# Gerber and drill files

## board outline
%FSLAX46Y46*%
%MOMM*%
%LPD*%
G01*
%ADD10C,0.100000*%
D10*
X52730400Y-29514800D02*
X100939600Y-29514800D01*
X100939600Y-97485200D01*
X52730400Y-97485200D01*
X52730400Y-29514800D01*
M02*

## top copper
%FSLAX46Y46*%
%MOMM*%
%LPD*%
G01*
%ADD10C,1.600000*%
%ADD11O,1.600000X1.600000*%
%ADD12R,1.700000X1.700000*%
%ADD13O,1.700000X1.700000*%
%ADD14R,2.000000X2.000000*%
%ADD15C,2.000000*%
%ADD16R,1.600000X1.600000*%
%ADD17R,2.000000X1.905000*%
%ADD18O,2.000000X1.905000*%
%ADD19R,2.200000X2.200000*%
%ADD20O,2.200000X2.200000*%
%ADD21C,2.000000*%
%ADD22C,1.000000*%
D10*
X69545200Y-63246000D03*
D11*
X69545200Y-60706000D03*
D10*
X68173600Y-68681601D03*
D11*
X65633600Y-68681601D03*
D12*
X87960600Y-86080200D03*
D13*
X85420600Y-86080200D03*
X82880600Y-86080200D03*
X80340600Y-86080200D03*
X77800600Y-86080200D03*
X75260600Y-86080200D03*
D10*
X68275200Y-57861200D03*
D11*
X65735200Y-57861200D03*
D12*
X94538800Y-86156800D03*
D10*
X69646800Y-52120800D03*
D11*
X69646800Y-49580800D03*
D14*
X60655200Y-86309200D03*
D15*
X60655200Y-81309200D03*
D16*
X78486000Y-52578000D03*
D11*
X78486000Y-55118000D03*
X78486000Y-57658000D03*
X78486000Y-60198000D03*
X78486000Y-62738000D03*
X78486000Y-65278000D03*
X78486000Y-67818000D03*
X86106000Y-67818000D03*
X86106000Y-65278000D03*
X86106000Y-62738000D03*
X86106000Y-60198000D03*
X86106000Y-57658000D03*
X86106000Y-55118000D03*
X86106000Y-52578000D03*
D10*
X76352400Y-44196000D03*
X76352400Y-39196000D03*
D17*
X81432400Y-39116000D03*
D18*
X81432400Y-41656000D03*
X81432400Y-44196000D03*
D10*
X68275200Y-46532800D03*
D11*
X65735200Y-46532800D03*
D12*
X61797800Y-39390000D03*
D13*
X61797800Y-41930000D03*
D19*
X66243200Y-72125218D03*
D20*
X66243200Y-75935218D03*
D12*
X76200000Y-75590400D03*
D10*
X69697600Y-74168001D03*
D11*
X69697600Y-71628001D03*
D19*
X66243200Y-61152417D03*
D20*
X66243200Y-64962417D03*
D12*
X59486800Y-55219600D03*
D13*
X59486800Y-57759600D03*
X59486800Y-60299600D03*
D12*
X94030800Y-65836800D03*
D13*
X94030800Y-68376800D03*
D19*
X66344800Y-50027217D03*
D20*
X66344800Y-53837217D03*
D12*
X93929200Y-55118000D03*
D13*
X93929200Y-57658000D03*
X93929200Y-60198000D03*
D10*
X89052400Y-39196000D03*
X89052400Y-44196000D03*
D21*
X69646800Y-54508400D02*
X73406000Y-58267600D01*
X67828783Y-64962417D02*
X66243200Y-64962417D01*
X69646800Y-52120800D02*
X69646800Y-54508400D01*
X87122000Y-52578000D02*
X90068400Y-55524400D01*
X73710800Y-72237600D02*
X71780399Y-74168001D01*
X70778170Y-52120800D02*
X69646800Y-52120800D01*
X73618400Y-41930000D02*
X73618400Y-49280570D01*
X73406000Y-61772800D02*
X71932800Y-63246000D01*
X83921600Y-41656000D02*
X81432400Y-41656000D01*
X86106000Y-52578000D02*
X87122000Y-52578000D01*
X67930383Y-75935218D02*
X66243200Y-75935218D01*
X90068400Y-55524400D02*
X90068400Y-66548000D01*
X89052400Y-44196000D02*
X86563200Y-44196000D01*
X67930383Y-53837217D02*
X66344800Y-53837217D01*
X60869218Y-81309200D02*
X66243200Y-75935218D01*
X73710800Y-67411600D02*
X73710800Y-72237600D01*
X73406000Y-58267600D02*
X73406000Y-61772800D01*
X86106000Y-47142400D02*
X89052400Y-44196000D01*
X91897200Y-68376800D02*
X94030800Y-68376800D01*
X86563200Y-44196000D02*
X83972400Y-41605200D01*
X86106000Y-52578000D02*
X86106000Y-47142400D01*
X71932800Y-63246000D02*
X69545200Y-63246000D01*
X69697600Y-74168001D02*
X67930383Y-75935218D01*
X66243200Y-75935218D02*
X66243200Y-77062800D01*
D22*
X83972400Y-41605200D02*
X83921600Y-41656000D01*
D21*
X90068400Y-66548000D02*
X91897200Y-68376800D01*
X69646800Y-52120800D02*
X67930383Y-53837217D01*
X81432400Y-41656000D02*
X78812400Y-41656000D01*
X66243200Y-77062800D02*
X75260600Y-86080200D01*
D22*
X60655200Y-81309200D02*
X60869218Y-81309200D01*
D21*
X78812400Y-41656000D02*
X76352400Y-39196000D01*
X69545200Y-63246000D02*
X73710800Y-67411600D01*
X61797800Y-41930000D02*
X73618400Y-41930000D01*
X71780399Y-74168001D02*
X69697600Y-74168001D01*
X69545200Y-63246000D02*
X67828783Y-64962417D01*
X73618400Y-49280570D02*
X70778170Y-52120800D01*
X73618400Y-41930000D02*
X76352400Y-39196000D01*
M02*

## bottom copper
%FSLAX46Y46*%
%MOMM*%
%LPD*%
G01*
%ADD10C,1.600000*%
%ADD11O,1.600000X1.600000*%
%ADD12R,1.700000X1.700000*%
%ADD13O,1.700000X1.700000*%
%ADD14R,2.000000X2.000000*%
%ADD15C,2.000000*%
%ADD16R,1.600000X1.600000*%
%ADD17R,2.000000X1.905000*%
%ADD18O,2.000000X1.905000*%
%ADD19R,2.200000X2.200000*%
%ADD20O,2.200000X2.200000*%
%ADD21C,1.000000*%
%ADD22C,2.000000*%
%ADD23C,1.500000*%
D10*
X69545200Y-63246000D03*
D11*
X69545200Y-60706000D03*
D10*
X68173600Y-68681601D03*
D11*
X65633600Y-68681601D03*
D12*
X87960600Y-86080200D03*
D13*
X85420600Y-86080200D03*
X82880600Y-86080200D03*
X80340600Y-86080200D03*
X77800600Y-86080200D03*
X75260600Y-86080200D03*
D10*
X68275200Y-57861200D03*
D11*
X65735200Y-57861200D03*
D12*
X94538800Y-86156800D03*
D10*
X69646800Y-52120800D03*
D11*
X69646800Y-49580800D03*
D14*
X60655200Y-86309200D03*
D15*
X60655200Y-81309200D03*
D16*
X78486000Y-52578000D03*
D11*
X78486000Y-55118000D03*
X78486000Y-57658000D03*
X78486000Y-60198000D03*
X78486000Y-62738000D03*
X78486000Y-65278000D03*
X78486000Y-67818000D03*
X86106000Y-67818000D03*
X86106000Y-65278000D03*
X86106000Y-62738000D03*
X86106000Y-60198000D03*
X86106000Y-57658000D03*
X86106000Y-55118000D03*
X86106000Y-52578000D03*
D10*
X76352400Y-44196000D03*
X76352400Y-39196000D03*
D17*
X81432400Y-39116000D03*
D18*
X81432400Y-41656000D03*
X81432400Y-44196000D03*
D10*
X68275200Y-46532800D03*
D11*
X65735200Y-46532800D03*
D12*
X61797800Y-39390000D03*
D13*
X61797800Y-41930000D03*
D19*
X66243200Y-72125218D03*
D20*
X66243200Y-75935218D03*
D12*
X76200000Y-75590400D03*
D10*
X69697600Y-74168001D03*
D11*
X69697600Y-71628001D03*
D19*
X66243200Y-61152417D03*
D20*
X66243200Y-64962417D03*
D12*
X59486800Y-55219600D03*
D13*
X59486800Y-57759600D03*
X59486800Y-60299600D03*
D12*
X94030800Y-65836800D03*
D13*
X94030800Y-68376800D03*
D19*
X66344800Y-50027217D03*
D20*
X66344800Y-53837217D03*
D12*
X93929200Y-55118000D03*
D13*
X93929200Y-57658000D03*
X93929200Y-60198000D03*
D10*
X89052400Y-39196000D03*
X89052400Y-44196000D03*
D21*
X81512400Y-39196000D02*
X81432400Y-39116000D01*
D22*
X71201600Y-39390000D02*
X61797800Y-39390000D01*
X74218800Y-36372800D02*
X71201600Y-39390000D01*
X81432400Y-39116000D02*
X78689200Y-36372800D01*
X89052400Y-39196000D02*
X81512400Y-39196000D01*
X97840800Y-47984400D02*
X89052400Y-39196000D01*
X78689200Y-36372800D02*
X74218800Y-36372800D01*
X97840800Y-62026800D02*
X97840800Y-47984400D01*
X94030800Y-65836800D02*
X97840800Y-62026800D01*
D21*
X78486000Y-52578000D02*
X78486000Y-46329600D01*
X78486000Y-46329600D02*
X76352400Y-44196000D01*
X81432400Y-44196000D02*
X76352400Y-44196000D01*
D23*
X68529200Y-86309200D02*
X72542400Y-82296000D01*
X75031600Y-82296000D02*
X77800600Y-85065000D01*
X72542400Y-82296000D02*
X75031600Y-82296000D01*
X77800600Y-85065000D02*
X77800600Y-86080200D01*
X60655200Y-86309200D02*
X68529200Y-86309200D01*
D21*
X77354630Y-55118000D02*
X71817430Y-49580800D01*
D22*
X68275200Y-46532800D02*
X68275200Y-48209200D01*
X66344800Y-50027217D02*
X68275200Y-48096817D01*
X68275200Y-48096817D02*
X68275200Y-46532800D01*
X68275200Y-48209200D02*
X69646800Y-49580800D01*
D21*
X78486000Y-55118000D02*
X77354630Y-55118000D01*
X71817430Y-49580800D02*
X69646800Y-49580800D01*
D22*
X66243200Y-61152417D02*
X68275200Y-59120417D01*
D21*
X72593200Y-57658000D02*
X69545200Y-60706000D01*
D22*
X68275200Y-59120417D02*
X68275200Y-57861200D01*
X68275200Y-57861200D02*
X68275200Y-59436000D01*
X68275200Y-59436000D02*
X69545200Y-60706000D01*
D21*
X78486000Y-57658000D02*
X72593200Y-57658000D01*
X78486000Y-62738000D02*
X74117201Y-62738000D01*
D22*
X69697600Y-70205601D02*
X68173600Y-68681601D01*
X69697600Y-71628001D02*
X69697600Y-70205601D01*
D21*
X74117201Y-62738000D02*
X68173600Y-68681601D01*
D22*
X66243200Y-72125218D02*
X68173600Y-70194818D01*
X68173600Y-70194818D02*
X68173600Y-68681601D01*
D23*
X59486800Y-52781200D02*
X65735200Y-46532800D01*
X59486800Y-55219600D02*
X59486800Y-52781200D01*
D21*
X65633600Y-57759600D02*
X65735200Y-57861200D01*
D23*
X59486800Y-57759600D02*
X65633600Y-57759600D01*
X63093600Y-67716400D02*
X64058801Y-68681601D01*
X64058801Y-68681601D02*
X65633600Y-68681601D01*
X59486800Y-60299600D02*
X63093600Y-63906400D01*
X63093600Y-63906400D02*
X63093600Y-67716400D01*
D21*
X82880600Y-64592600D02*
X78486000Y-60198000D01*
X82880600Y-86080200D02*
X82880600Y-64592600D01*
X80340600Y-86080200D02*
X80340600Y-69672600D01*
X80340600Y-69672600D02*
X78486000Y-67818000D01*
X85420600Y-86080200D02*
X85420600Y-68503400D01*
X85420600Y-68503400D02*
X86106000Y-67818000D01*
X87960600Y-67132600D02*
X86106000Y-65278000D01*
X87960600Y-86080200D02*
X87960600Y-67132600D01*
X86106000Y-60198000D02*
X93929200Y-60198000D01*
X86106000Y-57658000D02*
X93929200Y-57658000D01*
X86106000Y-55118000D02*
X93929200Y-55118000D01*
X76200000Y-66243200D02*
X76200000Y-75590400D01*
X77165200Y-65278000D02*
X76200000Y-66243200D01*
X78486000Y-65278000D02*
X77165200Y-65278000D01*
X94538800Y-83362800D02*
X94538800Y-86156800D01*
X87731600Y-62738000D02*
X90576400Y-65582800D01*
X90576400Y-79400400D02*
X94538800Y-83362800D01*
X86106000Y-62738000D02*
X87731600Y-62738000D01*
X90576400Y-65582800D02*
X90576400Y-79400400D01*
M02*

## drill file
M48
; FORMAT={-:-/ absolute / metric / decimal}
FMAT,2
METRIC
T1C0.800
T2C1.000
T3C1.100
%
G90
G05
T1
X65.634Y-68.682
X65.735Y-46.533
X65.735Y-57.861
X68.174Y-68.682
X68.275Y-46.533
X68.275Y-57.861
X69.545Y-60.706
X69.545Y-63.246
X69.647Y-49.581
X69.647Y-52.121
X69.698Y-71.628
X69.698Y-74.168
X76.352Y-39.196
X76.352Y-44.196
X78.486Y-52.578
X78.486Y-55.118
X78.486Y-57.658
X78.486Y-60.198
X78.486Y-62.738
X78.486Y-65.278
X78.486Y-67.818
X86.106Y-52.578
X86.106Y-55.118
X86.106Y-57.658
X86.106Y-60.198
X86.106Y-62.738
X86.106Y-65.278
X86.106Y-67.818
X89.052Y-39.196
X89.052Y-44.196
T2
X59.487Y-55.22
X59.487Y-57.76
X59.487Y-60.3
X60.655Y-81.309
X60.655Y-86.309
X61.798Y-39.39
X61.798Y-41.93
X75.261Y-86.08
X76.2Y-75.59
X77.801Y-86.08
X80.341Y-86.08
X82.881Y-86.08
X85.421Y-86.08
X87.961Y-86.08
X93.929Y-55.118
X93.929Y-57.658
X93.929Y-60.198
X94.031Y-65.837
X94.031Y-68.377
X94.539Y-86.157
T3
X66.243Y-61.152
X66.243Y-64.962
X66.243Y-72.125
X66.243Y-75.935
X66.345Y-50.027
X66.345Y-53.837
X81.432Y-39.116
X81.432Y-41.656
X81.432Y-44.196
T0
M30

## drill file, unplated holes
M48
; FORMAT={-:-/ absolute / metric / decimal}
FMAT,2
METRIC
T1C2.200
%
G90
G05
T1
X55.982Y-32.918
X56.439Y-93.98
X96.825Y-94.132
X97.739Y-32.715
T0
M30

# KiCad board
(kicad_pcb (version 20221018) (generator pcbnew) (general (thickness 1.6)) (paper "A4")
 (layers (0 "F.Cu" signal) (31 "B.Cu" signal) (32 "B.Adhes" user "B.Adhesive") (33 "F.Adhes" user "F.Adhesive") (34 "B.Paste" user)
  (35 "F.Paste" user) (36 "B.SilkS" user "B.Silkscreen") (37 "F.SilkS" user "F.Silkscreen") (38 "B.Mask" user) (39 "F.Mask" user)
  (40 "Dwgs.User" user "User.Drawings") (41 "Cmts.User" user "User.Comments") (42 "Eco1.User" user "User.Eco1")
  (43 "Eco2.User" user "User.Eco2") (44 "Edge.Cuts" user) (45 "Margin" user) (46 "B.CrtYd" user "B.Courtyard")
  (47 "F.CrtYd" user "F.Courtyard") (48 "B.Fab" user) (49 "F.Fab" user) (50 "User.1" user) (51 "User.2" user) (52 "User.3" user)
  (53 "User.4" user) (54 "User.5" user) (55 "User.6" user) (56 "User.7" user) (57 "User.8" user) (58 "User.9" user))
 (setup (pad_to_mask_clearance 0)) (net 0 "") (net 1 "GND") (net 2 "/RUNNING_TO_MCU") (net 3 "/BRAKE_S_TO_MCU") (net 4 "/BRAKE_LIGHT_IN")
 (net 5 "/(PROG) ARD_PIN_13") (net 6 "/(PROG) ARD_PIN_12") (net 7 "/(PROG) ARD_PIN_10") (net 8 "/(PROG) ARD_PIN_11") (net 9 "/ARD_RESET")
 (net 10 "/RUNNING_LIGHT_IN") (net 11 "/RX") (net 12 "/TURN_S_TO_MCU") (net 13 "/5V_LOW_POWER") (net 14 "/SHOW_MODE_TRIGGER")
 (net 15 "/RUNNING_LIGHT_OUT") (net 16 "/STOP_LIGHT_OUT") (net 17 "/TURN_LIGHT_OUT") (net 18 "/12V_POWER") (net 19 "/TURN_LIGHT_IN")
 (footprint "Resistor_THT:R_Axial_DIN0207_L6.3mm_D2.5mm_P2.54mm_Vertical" (layer "F.Cu") (at 69.5452 63.246 90)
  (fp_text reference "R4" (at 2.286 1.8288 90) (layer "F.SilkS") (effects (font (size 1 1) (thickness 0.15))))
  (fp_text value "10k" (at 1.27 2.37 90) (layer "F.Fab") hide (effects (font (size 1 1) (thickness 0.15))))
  (pad "1" thru_hole circle (at 0 0 90) (size 1.6 1.6) (drill 0.8) (layers "*.Cu" "*.Mask") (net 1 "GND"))
  (pad "2" thru_hole oval (at 2.54 0 90) (size 1.6 1.6) (drill 0.8) (layers "*.Cu" "*.Mask") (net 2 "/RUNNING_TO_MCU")))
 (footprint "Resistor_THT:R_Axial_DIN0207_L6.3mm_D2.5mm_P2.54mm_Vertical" (layer "F.Cu") (at 68.1736 68.681601 180)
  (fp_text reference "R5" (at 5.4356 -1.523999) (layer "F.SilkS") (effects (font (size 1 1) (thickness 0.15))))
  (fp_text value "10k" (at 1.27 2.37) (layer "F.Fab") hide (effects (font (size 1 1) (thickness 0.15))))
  (pad "1" thru_hole circle (at 0 0 180) (size 1.6 1.6) (drill 0.8) (layers "*.Cu" "*.Mask") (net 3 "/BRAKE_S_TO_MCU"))
  (pad "2" thru_hole oval (at 2.54 0 180) (size 1.6 1.6) (drill 0.8) (layers "*.Cu" "*.Mask") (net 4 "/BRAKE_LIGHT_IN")))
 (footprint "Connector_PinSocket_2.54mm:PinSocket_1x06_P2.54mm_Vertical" (layer "F.Cu") (at 87.9606 86.0802 -90)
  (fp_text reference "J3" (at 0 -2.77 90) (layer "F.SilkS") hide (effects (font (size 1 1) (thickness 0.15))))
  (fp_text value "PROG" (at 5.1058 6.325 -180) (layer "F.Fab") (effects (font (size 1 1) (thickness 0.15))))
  (pad "1" thru_hole rect (at 0 0 270) (size 1.7 1.7) (drill 1) (layers "*.Cu" "*.Mask") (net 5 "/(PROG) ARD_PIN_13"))
  (pad "2" thru_hole oval (at 0 2.54 270) (size 1.7 1.7) (drill 1) (layers "*.Cu" "*.Mask") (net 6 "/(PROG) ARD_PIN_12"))
  (pad "3" thru_hole oval (at 0 5.08 270) (size 1.7 1.7) (drill 1) (layers "*.Cu" "*.Mask") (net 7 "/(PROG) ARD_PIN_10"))
  (pad "4" thru_hole oval (at 0 7.62 270) (size 1.7 1.7) (drill 1) (layers "*.Cu" "*.Mask") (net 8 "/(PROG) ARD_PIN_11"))
  (pad "5" thru_hole oval (at 0 10.16 270) (size 1.7 1.7) (drill 1) (layers "*.Cu" "*.Mask") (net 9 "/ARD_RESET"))
  (pad "6" thru_hole oval (at 0 12.7 270) (size 1.7 1.7) (drill 1) (layers "*.Cu" "*.Mask") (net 1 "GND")))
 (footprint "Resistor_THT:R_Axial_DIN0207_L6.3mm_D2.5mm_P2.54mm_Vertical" (layer "F.Cu") (at 68.2752 57.8612 180)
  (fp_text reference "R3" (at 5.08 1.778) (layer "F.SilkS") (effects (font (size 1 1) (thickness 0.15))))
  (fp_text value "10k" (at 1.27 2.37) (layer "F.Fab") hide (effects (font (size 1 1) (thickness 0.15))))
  (pad "1" thru_hole circle (at 0 0 180) (size 1.6 1.6) (drill 0.8) (layers "*.Cu" "*.Mask") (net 2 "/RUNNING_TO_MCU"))
  (pad "2" thru_hole oval (at 2.54 0 180) (size 1.6 1.6) (drill 0.8) (layers "*.Cu" "*.Mask") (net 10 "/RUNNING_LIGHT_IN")))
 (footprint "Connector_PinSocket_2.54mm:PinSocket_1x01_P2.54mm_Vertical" (layer "F.Cu") (at 94.5388 86.1568)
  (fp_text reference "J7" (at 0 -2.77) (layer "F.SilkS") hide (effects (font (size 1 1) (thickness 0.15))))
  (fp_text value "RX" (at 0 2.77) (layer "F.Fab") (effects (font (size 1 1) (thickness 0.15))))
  (pad "1" thru_hole rect (at 0 0) (size 1.7 1.7) (drill 1) (layers "*.Cu" "*.Mask") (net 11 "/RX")))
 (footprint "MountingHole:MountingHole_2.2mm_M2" (layer "F.Cu") (at 96.8248 94.1324)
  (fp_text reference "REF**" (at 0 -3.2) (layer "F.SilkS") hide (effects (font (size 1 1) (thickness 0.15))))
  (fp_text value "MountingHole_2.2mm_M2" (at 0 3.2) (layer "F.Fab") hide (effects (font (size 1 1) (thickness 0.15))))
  (pad "" np_thru_hole circle (at 0 0) (size 2.2 2.2) (drill 2.2) (layers "*.Cu" "*.Mask")))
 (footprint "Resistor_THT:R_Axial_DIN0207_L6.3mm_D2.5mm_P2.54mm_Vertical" (layer "F.Cu") (at 69.6468 52.1208 90)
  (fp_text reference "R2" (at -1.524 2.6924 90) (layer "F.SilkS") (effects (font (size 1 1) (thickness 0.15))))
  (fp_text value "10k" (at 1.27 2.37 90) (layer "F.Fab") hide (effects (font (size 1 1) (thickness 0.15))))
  (pad "1" thru_hole circle (at 0 0 90) (size 1.6 1.6) (drill 0.8) (layers "*.Cu" "*.Mask") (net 1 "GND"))
  (pad "2" thru_hole oval (at 2.54 0 90) (size 1.6 1.6) (drill 0.8) (layers "*.Cu" "*.Mask") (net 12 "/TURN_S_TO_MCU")))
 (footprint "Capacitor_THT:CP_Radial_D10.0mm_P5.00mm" (layer "F.Cu") (at 60.6552 86.3092 90)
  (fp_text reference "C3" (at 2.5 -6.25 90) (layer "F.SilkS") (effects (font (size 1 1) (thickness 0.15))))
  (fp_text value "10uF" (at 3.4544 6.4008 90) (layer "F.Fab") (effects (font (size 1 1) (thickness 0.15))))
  (pad "1" thru_hole rect (at 0 0 90) (size 2 2) (drill 1) (layers "*.Cu" "*.Mask") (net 9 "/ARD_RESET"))
  (pad "2" thru_hole circle (at 5 0 90) (size 2 2) (drill 1) (layers "*.Cu" "*.Mask") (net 1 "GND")))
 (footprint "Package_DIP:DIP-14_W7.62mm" (layer "F.Cu") (at 78.486 52.578)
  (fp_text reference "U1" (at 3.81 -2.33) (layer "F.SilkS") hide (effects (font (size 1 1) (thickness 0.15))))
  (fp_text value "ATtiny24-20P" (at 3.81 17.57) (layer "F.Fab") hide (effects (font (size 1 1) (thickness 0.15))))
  (pad "1" thru_hole rect (at 0 0) (size 1.6 1.6) (drill 0.8) (layers "*.Cu" "*.Mask") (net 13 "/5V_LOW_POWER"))
  (pad "2" thru_hole oval (at 0 2.54) (size 1.6 1.6) (drill 0.8) (layers "*.Cu" "*.Mask") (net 12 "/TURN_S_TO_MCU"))
  (pad "3" thru_hole oval (at 0 5.08) (size 1.6 1.6) (drill 0.8) (layers "*.Cu" "*.Mask") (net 2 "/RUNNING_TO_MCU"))
  (pad "4" thru_hole oval (at 0 7.62) (size 1.6 1.6) (drill 0.8) (layers "*.Cu" "*.Mask") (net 7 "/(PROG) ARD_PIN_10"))
  (pad "5" thru_hole oval (at 0 10.16) (size 1.6 1.6) (drill 0.8) (layers "*.Cu" "*.Mask") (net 3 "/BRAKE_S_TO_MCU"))
  (pad "6" thru_hole oval (at 0 12.7) (size 1.6 1.6) (drill 0.8) (layers "*.Cu" "*.Mask") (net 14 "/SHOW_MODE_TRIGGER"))
  (pad "7" thru_hole oval (at 0 15.24) (size 1.6 1.6) (drill 0.8) (layers "*.Cu" "*.Mask") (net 8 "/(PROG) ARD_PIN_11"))
  (pad "8" thru_hole oval (at 7.62 15.24) (size 1.6 1.6) (drill 0.8) (layers "*.Cu" "*.Mask") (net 6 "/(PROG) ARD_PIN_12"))
  (pad "9" thru_hole oval (at 7.62 12.7) (size 1.6 1.6) (drill 0.8) (layers "*.Cu" "*.Mask") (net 5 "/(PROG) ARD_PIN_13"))
  (pad "10" thru_hole oval (at 7.62 10.16) (size 1.6 1.6) (drill 0.8) (layers "*.Cu" "*.Mask") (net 11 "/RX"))
  (pad "11" thru_hole oval (at 7.62 7.62) (size 1.6 1.6) (drill 0.8) (layers "*.Cu" "*.Mask") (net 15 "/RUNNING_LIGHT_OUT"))
  (pad "12" thru_hole oval (at 7.62 5.08) (size 1.6 1.6) (drill 0.8) (layers "*.Cu" "*.Mask") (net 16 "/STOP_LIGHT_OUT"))
  (pad "13" thru_hole oval (at 7.62 2.54) (size 1.6 1.6) (drill 0.8) (layers "*.Cu" "*.Mask") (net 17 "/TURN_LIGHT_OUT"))
  (pad "14" thru_hole oval (at 7.62 0) (size 1.6 1.6) (drill 0.8) (layers "*.Cu" "*.Mask") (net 1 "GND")))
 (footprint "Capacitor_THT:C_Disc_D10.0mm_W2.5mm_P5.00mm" (layer "F.Cu") (at 76.3524 44.196 90)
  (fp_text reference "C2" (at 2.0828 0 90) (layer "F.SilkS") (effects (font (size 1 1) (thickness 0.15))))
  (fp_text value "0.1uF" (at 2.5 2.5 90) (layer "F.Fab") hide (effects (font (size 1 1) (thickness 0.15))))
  (pad "1" thru_hole circle (at 0 0 90) (size 1.6 1.6) (drill 0.8) (layers "*.Cu" "*.Mask") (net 13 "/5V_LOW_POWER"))
  (pad "2" thru_hole circle (at 5 0 90) (size 1.6 1.6) (drill 0.8) (layers "*.Cu" "*.Mask") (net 1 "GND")))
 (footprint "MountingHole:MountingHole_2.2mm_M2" (layer "F.Cu") (at 56.4388 93.98)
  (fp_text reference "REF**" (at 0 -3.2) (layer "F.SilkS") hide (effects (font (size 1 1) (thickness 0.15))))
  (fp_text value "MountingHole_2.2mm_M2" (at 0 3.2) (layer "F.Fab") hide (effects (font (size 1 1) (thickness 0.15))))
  (pad "" np_thru_hole circle (at 0 0) (size 2.2 2.2) (drill 2.2) (layers "*.Cu" "*.Mask")))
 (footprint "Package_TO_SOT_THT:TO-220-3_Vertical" (layer "F.Cu") (at 81.4324 39.116 -90)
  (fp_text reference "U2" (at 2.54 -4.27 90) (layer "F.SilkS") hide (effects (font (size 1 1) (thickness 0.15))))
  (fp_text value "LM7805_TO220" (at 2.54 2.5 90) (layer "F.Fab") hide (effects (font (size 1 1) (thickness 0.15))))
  (pad "1" thru_hole rect (at 0 0 270) (size 1.905 2) (drill 1.1) (layers "*.Cu" "*.Mask") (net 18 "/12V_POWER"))
  (pad "2" thru_hole oval (at 2.54 0 270) (size 1.905 2) (drill 1.1) (layers "*.Cu" "*.Mask") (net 1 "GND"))
  (pad "3" thru_hole oval (at 5.08 0 270) (size 1.905 2) (drill 1.1) (layers "*.Cu" "*.Mask") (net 13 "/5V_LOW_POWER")))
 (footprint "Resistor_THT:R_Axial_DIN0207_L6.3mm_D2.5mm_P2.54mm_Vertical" (layer "F.Cu") (at 68.2752 46.5328 180)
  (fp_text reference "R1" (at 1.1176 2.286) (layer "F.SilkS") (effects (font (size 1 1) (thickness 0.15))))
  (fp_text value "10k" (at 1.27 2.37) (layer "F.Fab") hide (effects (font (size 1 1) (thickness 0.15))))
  (pad "1" thru_hole circle (at 0 0 180) (size 1.6 1.6) (drill 0.8) (layers "*.Cu" "*.Mask") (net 12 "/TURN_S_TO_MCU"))
  (pad "2" thru_hole oval (at 2.54 0 180) (size 1.6 1.6) (drill 0.8) (layers "*.Cu" "*.Mask") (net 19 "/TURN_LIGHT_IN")))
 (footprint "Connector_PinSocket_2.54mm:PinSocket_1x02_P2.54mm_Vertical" (layer "F.Cu") (at 61.7978 39.39)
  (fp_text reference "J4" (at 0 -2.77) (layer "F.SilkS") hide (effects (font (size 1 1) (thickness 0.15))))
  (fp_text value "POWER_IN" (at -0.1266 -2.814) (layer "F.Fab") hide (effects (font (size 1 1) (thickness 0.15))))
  (pad "1" thru_hole rect (at 0 0) (size 1.7 1.7) (drill 1) (layers "*.Cu" "*.Mask") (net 18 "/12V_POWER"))
  (pad "2" thru_hole oval (at 0 2.54) (size 1.7 1.7) (drill 1) (layers "*.Cu" "*.Mask") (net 1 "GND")))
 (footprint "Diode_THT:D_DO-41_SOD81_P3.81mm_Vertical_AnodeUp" (layer "F.Cu") (at 66.2432 72.125218 -90)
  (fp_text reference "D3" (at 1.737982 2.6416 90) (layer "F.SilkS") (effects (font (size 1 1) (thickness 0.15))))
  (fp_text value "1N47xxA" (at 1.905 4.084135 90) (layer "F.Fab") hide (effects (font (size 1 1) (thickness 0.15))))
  (pad "1" thru_hole rect (at 0 0 270) (size 2.2 2.2) (drill 1.1) (layers "*.Cu" "*.Mask") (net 3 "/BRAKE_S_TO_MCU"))
  (pad "2" thru_hole oval (at 3.81 0 270) (size 2.2 2.2) (drill 1.1) (layers "*.Cu" "*.Mask") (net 1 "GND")))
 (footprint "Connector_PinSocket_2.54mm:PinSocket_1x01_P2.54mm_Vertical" (layer "F.Cu") (at 76.2 75.5904)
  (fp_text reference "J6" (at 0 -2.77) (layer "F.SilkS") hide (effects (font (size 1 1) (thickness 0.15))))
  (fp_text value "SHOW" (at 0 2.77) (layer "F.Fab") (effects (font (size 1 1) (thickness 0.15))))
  (pad "1" thru_hole rect (at 0 0) (size 1.7 1.7) (drill 1) (layers "*.Cu" "*.Mask") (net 14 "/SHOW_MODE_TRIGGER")))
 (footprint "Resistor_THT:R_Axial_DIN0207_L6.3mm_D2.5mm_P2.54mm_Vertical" (layer "F.Cu") (at 69.6976 74.168001 90)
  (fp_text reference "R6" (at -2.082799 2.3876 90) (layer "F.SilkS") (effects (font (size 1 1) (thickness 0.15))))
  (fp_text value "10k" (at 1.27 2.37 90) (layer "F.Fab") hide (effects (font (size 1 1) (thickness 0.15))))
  (pad "1" thru_hole circle (at 0 0 90) (size 1.6 1.6) (drill 0.8) (layers "*.Cu" "*.Mask") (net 1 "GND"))
  (pad "2" thru_hole oval (at 2.54 0 90) (size 1.6 1.6) (drill 0.8) (layers "*.Cu" "*.Mask") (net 3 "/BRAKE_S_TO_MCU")))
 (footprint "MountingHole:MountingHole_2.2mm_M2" (layer "F.Cu") (at 55.9816 32.9184)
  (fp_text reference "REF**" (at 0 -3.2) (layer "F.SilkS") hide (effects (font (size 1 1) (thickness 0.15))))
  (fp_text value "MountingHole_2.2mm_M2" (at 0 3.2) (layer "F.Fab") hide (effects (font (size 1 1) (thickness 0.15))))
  (pad "" np_thru_hole circle (at 0 0) (size 2.2 2.2) (drill 2.2) (layers "*.Cu" "*.Mask")))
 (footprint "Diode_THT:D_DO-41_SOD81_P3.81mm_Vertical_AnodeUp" (layer "F.Cu") (at 66.2432 61.152417 -90)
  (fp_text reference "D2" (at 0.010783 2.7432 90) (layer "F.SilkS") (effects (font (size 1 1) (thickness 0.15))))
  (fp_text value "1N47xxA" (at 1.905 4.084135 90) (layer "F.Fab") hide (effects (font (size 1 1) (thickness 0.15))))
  (pad "1" thru_hole rect (at 0 0 270) (size 2.2 2.2) (drill 1.1) (layers "*.Cu" "*.Mask") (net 2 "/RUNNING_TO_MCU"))
  (pad "2" thru_hole oval (at 3.81 0 270) (size 2.2 2.2) (drill 1.1) (layers "*.Cu" "*.Mask") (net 1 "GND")))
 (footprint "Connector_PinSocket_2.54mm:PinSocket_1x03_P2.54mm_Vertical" (layer "F.Cu") (at 59.4868 55.2196)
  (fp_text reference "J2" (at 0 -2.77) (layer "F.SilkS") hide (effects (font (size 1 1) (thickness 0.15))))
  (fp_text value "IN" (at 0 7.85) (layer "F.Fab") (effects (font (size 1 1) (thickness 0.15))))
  (pad "1" thru_hole rect (at 0 0) (size 1.7 1.7) (drill 1) (layers "*.Cu" "*.Mask") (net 19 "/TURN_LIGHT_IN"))
  (pad "2" thru_hole oval (at 0 2.54) (size 1.7 1.7) (drill 1) (layers "*.Cu" "*.Mask") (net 10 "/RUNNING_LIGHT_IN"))
  (pad "3" thru_hole oval (at 0 5.08) (size 1.7 1.7) (drill 1) (layers "*.Cu" "*.Mask") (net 4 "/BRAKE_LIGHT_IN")))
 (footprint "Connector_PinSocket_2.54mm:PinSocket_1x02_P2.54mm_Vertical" (layer "F.Cu") (at 94.0308 65.8368)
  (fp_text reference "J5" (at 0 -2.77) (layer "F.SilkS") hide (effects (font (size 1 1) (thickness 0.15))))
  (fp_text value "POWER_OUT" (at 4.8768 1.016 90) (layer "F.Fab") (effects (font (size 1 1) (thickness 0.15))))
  (pad "1" thru_hole rect (at 0 0) (size 1.7 1.7) (drill 1) (layers "*.Cu" "*.Mask") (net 18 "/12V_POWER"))
  (pad "2" thru_hole oval (at 0 2.54) (size 1.7 1.7) (drill 1) (layers "*.Cu" "*.Mask") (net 1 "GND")))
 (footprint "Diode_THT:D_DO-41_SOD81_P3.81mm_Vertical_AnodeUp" (layer "F.Cu") (at 66.3448 50.027217 -90)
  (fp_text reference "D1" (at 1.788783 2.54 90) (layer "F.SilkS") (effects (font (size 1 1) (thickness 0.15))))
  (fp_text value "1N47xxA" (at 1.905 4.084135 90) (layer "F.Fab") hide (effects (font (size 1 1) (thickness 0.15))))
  (pad "1" thru_hole rect (at 0 0 270) (size 2.2 2.2) (drill 1.1) (layers "*.Cu" "*.Mask") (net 12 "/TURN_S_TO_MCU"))
  (pad "2" thru_hole oval (at 3.81 0 270) (size 2.2 2.2) (drill 1.1) (layers "*.Cu" "*.Mask") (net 1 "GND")))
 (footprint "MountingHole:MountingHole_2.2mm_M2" (layer "F.Cu") (at 97.7392 32.7152)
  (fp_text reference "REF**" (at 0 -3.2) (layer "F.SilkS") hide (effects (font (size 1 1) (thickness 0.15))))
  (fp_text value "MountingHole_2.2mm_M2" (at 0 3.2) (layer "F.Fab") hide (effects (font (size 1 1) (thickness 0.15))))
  (pad "" np_thru_hole circle (at 0 0) (size 2.2 2.2) (drill 2.2) (layers "*.Cu" "*.Mask")))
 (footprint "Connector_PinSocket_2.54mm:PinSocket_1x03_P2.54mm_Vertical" (layer "F.Cu") (at 93.9292 55.118)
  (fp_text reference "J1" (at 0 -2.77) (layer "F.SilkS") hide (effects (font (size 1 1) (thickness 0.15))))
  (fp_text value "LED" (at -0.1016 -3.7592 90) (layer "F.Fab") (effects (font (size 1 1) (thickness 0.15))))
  (pad "1" thru_hole rect (at 0 0) (size 1.7 1.7) (drill 1) (layers "*.Cu" "*.Mask") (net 17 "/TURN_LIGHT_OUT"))
  (pad "2" thru_hole oval (at 0 2.54) (size 1.7 1.7) (drill 1) (layers "*.Cu" "*.Mask") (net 16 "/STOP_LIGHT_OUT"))
  (pad "3" thru_hole oval (at 0 5.08) (size 1.7 1.7) (drill 1) (layers "*.Cu" "*.Mask") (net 15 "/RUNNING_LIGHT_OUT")))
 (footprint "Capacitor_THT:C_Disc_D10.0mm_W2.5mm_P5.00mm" (layer "F.Cu") (at 89.0524 39.196 -90)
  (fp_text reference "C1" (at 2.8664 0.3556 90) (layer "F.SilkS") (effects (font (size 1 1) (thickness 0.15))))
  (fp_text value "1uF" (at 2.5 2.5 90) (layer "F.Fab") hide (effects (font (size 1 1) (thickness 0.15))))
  (pad "1" thru_hole circle (at 0 0 270) (size 1.6 1.6) (drill 0.8) (layers "*.Cu" "*.Mask") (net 18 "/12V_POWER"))
  (pad "2" thru_hole circle (at 5 0 270) (size 1.6 1.6) (drill 0.8) (layers "*.Cu" "*.Mask") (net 1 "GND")))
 (gr_rect (start 52.7304 29.5148) (end 100.9396 97.4852) (stroke (width 0.1) (type default)) (fill none) (layer "Edge.Cuts"))
 (segment (start 81.5124 39.196) (end 81.4324 39.116) (width 1) (layer "B.Cu") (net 18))
 (segment (start 71.2016 39.39) (end 61.7978 39.39) (width 2) (layer "B.Cu") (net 18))
 (segment (start 74.2188 36.3728) (end 71.2016 39.39) (width 2) (layer "B.Cu") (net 18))
 (segment (start 81.4324 39.116) (end 78.6892 36.3728) (width 2) (layer "B.Cu") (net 18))
 (segment (start 89.0524 39.196) (end 81.5124 39.196) (width 2) (layer "B.Cu") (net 18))
 (segment (start 97.8408 47.9844) (end 89.0524 39.196) (width 2) (layer "B.Cu") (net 18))
 (segment (start 78.6892 36.3728) (end 74.2188 36.3728) (width 2) (layer "B.Cu") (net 18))
 (segment (start 97.8408 62.0268) (end 97.8408 47.9844) (width 2) (layer "B.Cu") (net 18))
 (segment (start 94.0308 65.8368) (end 97.8408 62.0268) (width 2) (layer "B.Cu") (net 18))
 (segment (start 69.6468 54.5084) (end 73.406 58.2676) (width 2) (layer "F.Cu") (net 1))
 (segment (start 67.828783 64.962417) (end 66.2432 64.962417) (width 2) (layer "F.Cu") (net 1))
 (segment (start 69.6468 52.1208) (end 69.6468 54.5084) (width 2) (layer "F.Cu") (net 1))
 (segment (start 87.122 52.578) (end 90.0684 55.5244) (width 2) (layer "F.Cu") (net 1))
 (segment (start 73.7108 72.2376) (end 71.780399 74.168001) (width 2) (layer "F.Cu") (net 1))
 (segment (start 70.77817 52.1208) (end 69.6468 52.1208) (width 2) (layer "F.Cu") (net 1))
 (segment (start 73.6184 41.93) (end 73.6184 49.28057) (width 2) (layer "F.Cu") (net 1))
 (segment (start 73.406 61.7728) (end 71.9328 63.246) (width 2) (layer "F.Cu") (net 1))
 (segment (start 83.9216 41.656) (end 81.4324 41.656) (width 2) (layer "F.Cu") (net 1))
 (segment (start 86.106 52.578) (end 87.122 52.578) (width 2) (layer "F.Cu") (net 1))
 (segment (start 67.930383 75.935218) (end 66.2432 75.935218) (width 2) (layer "F.Cu") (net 1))
 (segment (start 90.0684 55.5244) (end 90.0684 66.548) (width 2) (layer "F.Cu") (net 1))
 (segment (start 89.0524 44.196) (end 86.5632 44.196) (width 2) (layer "F.Cu") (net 1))
 (segment (start 67.930383 53.837217) (end 66.3448 53.837217) (width 2) (layer "F.Cu") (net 1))
 (segment (start 60.869218 81.3092) (end 66.2432 75.935218) (width 2) (layer "F.Cu") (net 1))
 (segment (start 73.7108 67.4116) (end 73.7108 72.2376) (width 2) (layer "F.Cu") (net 1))
 (segment (start 73.406 58.2676) (end 73.406 61.7728) (width 2) (layer "F.Cu") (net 1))
 (segment (start 86.106 47.1424) (end 89.0524 44.196) (width 2) (layer "F.Cu") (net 1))
 (segment (start 91.8972 68.3768) (end 94.0308 68.3768) (width 2) (layer "F.Cu") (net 1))
 (segment (start 86.5632 44.196) (end 83.9724 41.6052) (width 2) (layer "F.Cu") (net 1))
 (segment (start 86.106 52.578) (end 86.106 47.1424) (width 2) (layer "F.Cu") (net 1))
 (segment (start 71.9328 63.246) (end 69.5452 63.246) (width 2) (layer "F.Cu") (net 1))
 (segment (start 69.6976 74.168001) (end 67.930383 75.935218) (width 2) (layer "F.Cu") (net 1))
 (segment (start 66.2432 75.935218) (end 66.2432 77.0628) (width 2) (layer "F.Cu") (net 1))
 (segment (start 83.9724 41.6052) (end 83.9216 41.656) (width 1) (layer "F.Cu") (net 1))
 (segment (start 90.0684 66.548) (end 91.8972 68.3768) (width 2) (layer "F.Cu") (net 1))
 (segment (start 69.6468 52.1208) (end 67.930383 53.837217) (width 2) (layer "F.Cu") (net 1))
 (segment (start 81.4324 41.656) (end 78.8124 41.656) (width 2) (layer "F.Cu") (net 1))
 (segment (start 66.2432 77.0628) (end 75.2606 86.0802) (width 2) (layer "F.Cu") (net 1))
 (segment (start 60.6552 81.3092) (end 60.869218 81.3092) (width 1) (layer "F.Cu") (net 1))
 (segment (start 78.8124 41.656) (end 76.3524 39.196) (width 2) (layer "F.Cu") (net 1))
 (segment (start 69.5452 63.246) (end 73.7108 67.4116) (width 2) (layer "F.Cu") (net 1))
 (segment (start 61.7978 41.93) (end 73.6184 41.93) (width 2) (layer "F.Cu") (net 1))
 (segment (start 71.780399 74.168001) (end 69.6976 74.168001) (width 2) (layer "F.Cu") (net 1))
 (segment (start 69.5452 63.246) (end 67.828783 64.962417) (width 2) (layer "F.Cu") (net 1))
 (segment (start 73.6184 49.28057) (end 70.77817 52.1208) (width 2) (layer "F.Cu") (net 1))
 (segment (start 73.6184 41.93) (end 76.3524 39.196) (width 2) (layer "F.Cu") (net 1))
 (segment (start 78.486 52.578) (end 78.486 46.3296) (width 1) (layer "B.Cu") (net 13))
 (segment (start 78.486 46.3296) (end 76.3524 44.196) (width 1) (layer "B.Cu") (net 13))
 (segment (start 81.4324 44.196) (end 76.3524 44.196) (width 1) (layer "B.Cu") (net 13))
 (segment (start 68.5292 86.3092) (end 72.5424 82.296) (width 1.5) (layer "B.Cu") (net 9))
 (segment (start 75.0316 82.296) (end 77.8006 85.065) (width 1.5) (layer "B.Cu") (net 9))
 (segment (start 72.5424 82.296) (end 75.0316 82.296) (width 1.5) (layer "B.Cu") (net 9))
 (segment (start 77.8006 85.065) (end 77.8006 86.0802) (width 1.5) (layer "B.Cu") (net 9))
 (segment (start 60.6552 86.3092) (end 68.5292 86.3092) (width 1.5) (layer "B.Cu") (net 9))
 (segment (start 77.35463 55.118) (end 71.81743 49.5808) (width 1) (layer "B.Cu") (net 12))
 (segment (start 68.2752 46.5328) (end 68.2752 48.2092) (width 2) (layer "B.Cu") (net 12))
 (segment (start 66.3448 50.027217) (end 68.2752 48.096817) (width 2) (layer "B.Cu") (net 12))
 (segment (start 68.2752 48.096817) (end 68.2752 46.5328) (width 2) (layer "B.Cu") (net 12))
 (segment (start 68.2752 48.2092) (end 69.6468 49.5808) (width 2) (layer "B.Cu") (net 12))
 (segment (start 78.486 55.118) (end 77.35463 55.118) (width 1) (layer "B.Cu") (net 12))
 (segment (start 71.81743 49.5808) (end 69.6468 49.5808) (width 1) (layer "B.Cu") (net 12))
 (segment (start 66.2432 61.152417) (end 68.2752 59.120417) (width 2) (layer "B.Cu") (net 2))
 (segment (start 72.5932 57.658) (end 69.5452 60.706) (width 1) (layer "B.Cu") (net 2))
 (segment (start 68.2752 59.120417) (end 68.2752 57.8612) (width 2) (layer "B.Cu") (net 2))
 (segment (start 68.2752 57.8612) (end 68.2752 59.436) (width 2) (layer "B.Cu") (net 2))
 (segment (start 68.2752 59.436) (end 69.5452 60.706) (width 2) (layer "B.Cu") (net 2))
 (segment (start 78.486 57.658) (end 72.5932 57.658) (width 1) (layer "B.Cu") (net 2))
 (segment (start 78.486 62.738) (end 74.117201 62.738) (width 1) (layer "B.Cu") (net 3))
 (segment (start 69.6976 70.205601) (end 68.1736 68.681601) (width 2) (layer "B.Cu") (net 3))
 (segment (start 69.6976 71.628001) (end 69.6976 70.205601) (width 2) (layer "B.Cu") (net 3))
 (segment (start 74.117201 62.738) (end 68.1736 68.681601) (width 1) (layer "B.Cu") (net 3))
 (segment (start 66.2432 72.125218) (end 68.1736 70.194818) (width 2) (layer "B.Cu") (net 3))
 (segment (start 68.1736 70.194818) (end 68.1736 68.681601) (width 2) (layer "B.Cu") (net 3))
 (segment (start 59.4868 52.7812) (end 65.7352 46.5328) (width 1.5) (layer "B.Cu") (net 19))
 (segment (start 59.4868 55.2196) (end 59.4868 52.7812) (width 1.5) (layer "B.Cu") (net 19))
 (segment (start 65.6336 57.7596) (end 65.7352 57.8612) (width 1) (layer "B.Cu") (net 10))
 (segment (start 59.4868 57.7596) (end 65.6336 57.7596) (width 1.5) (layer "B.Cu") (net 10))
 (segment (start 63.0936 67.7164) (end 64.058801 68.681601) (width 1.5) (layer "B.Cu") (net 4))
 (segment (start 64.058801 68.681601) (end 65.6336 68.681601) (width 1.5) (layer "B.Cu") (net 4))
 (segment (start 59.4868 60.2996) (end 63.0936 63.9064) (width 1.5) (layer "B.Cu") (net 4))
 (segment (start 63.0936 63.9064) (end 63.0936 67.7164) (width 1.5) (layer "B.Cu") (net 4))
 (segment (start 82.8806 64.5926) (end 78.486 60.198) (width 1) (layer "B.Cu") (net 7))
 (segment (start 82.8806 86.0802) (end 82.8806 64.5926) (width 1) (layer "B.Cu") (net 7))
 (segment (start 80.3406 86.0802) (end 80.3406 69.6726) (width 1) (layer "B.Cu") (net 8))
 (segment (start 80.3406 69.6726) (end 78.486 67.818) (width 1) (layer "B.Cu") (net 8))
 (segment (start 85.4206 86.0802) (end 85.4206 68.5034) (width 1) (layer "B.Cu") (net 6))
 (segment (start 85.4206 68.5034) (end 86.106 67.818) (width 1) (layer "B.Cu") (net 6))
 (segment (start 87.9606 67.1326) (end 86.106 65.278) (width 1) (layer "B.Cu") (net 5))
 (segment (start 87.9606 86.0802) (end 87.9606 67.1326) (width 1) (layer "B.Cu") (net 5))
 (segment (start 86.106 60.198) (end 93.9292 60.198) (width 1) (layer "B.Cu") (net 15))
 (segment (start 86.106 57.658) (end 93.9292 57.658) (width 1) (layer "B.Cu") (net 16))
 (segment (start 86.106 55.118) (end 93.9292 55.118) (width 1) (layer "B.Cu") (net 17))
 (segment (start 76.2 66.2432) (end 76.2 75.5904) (width 1) (layer "B.Cu") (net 14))
 (segment (start 77.1652 65.278) (end 76.2 66.2432) (width 1) (layer "B.Cu") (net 14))
 (segment (start 78.486 65.278) (end 77.1652 65.278) (width 1) (layer "B.Cu") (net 14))
 (segment (start 94.5388 83.3628) (end 94.5388 86.1568) (width 1) (layer "B.Cu") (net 11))
 (segment (start 87.7316 62.738) (end 90.5764 65.5828) (width 1) (layer "B.Cu") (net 11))
 (segment (start 90.5764 79.4004) (end 94.5388 83.3628) (width 1) (layer "B.Cu") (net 11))
 (segment (start 86.106 62.738) (end 87.7316 62.738) (width 1) (layer "B.Cu") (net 11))
 (segment (start 90.5764 65.5828) (end 90.5764 79.4004) (width 1) (layer "B.Cu") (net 11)))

